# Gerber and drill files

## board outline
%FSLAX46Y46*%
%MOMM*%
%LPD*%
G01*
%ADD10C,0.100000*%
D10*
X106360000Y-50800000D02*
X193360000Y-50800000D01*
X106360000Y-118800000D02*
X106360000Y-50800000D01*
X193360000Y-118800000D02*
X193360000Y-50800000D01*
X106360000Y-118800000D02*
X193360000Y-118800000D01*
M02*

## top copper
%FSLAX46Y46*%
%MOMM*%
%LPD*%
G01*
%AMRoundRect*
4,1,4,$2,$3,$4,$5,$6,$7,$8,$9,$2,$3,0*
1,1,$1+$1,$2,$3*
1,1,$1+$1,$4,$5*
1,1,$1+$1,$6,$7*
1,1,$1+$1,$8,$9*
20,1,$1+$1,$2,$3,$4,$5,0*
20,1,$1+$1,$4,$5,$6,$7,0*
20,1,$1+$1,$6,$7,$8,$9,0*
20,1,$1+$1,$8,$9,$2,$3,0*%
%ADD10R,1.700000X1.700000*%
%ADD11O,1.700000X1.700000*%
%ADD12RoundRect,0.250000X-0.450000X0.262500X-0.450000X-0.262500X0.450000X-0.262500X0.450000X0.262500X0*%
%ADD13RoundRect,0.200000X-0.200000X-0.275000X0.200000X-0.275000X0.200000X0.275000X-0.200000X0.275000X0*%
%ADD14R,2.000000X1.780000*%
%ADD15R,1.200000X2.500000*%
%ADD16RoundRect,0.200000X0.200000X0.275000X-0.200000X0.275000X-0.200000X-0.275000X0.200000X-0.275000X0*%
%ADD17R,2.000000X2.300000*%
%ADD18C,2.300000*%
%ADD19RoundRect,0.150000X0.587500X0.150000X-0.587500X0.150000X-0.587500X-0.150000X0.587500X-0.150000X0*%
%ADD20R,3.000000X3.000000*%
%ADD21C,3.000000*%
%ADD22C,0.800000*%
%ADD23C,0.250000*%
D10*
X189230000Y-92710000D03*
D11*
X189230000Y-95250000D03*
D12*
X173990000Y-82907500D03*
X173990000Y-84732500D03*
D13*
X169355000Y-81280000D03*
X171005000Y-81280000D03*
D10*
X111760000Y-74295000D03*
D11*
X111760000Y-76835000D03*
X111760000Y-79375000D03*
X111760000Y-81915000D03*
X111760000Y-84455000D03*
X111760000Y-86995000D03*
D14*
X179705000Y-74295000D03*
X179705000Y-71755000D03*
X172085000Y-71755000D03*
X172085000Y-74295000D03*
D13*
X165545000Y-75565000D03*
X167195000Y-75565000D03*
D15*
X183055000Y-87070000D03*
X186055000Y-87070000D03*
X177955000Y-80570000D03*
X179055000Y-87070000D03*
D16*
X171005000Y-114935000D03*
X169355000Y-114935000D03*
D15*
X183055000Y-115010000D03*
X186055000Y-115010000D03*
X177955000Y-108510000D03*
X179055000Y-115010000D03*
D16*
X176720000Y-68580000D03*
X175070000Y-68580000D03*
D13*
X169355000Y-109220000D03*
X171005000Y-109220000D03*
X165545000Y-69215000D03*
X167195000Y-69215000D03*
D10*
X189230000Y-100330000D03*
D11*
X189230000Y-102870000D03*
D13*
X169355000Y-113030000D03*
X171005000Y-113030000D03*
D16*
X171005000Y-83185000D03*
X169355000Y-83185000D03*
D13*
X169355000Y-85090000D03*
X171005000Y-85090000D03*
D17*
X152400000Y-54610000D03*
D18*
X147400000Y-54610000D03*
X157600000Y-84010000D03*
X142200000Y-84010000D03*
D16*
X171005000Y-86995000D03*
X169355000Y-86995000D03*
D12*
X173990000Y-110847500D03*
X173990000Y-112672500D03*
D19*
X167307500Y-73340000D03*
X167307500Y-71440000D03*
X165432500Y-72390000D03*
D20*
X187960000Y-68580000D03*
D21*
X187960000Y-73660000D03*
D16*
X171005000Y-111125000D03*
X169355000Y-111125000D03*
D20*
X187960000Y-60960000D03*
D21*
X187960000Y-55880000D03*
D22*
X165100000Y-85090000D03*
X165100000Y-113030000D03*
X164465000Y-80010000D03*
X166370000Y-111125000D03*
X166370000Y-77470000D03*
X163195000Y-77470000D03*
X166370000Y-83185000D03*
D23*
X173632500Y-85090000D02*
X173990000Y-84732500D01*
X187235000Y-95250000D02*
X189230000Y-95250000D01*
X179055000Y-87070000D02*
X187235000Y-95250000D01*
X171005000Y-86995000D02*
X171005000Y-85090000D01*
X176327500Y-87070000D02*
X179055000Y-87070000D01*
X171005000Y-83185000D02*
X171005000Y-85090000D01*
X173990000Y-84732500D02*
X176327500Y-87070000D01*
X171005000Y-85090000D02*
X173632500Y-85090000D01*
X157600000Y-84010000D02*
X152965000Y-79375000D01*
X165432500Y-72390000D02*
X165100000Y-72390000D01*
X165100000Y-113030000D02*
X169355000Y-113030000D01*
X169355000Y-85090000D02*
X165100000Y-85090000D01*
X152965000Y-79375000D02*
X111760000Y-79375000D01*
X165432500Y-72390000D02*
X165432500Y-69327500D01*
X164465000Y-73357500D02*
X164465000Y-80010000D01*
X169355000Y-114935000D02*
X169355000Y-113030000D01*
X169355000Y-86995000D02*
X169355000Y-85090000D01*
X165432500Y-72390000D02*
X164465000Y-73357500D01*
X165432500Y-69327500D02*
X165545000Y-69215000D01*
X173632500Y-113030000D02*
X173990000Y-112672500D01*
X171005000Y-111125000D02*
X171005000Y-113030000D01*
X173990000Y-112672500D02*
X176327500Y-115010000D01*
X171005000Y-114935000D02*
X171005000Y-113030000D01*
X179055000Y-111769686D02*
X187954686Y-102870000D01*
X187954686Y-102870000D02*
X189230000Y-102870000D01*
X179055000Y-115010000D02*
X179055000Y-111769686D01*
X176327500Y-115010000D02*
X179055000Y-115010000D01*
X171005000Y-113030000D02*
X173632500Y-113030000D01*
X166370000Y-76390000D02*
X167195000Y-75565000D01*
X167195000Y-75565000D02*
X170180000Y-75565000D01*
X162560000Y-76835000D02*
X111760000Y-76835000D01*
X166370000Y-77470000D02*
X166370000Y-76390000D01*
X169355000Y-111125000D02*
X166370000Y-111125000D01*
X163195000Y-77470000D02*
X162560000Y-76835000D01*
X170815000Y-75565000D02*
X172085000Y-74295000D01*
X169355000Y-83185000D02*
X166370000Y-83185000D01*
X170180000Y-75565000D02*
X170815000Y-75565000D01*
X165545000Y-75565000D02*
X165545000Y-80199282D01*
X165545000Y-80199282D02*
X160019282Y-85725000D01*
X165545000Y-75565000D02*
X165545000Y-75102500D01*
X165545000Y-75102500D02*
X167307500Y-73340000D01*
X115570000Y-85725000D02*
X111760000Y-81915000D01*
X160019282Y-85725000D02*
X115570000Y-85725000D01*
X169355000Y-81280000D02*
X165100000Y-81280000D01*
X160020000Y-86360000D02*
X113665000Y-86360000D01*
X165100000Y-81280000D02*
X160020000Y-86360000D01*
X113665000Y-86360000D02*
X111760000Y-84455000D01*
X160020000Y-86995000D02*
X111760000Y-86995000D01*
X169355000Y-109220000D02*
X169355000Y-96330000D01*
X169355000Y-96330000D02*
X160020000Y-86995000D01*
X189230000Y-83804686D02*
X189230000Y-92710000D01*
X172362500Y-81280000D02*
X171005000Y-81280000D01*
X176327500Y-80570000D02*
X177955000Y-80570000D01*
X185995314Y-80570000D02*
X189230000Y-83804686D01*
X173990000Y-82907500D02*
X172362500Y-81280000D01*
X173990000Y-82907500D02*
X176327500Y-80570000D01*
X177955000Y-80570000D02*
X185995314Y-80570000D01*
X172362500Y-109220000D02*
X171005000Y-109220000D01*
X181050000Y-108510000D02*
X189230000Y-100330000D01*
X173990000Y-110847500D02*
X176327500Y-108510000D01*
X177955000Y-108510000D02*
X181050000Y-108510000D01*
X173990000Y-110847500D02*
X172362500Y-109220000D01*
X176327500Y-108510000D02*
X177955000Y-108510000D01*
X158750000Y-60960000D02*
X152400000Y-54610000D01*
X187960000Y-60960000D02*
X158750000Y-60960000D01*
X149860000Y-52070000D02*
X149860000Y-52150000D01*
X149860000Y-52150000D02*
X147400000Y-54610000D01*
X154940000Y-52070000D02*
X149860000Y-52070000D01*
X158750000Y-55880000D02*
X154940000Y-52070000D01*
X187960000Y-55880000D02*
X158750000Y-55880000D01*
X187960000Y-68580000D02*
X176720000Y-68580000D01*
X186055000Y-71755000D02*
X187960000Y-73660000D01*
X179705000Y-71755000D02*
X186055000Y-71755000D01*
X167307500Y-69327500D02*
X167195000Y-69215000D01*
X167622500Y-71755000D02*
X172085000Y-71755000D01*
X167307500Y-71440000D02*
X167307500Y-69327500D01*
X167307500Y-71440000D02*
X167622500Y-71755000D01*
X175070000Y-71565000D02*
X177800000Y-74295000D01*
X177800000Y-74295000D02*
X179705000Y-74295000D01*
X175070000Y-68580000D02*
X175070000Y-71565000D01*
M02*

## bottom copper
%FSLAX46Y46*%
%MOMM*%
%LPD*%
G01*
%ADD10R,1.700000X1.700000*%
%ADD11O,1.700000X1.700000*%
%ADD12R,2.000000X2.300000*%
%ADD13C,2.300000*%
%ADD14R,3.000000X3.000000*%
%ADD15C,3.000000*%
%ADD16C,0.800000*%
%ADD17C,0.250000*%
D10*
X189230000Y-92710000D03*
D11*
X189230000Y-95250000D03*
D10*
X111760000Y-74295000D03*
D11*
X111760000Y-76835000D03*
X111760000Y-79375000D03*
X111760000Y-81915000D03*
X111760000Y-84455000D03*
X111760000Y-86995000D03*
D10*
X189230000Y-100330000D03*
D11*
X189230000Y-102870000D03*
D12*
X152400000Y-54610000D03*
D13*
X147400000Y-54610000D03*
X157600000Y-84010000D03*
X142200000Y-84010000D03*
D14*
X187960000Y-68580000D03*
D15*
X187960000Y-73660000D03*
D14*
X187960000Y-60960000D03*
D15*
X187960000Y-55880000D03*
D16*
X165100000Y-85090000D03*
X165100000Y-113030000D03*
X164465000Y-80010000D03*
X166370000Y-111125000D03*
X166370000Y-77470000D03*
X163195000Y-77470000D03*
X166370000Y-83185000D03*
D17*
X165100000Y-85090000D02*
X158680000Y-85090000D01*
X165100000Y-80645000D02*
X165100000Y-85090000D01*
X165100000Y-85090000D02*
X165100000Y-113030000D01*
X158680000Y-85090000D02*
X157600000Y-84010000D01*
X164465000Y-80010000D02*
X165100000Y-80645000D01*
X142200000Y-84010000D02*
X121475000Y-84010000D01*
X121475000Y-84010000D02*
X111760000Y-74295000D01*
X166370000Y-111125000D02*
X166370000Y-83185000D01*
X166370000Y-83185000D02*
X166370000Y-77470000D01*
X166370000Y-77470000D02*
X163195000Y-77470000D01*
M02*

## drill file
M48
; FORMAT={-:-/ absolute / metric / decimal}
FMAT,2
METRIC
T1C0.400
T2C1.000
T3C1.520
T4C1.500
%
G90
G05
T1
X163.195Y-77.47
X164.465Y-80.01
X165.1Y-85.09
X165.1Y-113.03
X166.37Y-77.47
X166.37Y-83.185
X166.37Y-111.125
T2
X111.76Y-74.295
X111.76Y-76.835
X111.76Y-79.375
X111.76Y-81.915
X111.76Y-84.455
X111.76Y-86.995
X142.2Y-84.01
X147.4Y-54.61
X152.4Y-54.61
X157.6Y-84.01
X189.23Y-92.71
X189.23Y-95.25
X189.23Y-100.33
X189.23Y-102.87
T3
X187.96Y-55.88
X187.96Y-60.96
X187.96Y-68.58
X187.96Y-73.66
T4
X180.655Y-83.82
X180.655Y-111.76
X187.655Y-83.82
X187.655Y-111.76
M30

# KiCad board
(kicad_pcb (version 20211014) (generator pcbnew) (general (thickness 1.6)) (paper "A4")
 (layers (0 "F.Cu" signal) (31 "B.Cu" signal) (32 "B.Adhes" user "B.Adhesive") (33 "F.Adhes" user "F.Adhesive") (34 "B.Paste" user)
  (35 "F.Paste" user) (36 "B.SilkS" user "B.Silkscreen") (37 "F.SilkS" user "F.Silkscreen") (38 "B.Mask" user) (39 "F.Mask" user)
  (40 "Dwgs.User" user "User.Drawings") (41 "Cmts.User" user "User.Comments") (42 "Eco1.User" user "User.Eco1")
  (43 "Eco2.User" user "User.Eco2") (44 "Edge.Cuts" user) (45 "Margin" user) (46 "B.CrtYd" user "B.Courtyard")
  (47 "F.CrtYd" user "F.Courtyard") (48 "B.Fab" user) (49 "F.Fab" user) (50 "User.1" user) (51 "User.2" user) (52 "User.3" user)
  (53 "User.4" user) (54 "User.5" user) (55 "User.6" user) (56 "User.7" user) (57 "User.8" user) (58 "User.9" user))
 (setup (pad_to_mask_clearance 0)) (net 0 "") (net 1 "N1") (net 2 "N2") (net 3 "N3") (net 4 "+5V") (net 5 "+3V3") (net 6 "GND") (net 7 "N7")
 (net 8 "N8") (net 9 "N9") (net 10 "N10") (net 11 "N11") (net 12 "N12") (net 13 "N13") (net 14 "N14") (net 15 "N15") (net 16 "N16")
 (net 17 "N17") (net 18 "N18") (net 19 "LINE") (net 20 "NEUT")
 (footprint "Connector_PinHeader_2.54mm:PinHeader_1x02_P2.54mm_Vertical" (layer "F.Cu") (at 189.23 92.71)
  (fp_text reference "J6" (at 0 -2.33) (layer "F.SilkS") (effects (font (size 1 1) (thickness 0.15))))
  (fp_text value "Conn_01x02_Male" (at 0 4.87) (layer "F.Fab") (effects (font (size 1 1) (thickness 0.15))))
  (pad "1" thru_hole rect locked (at 0 0) (size 1.7 1.7) (drill 1) (layers *.Cu *.Mask) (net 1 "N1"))
  (pad "2" thru_hole oval locked (at 0 2.54) (size 1.7 1.7) (drill 1) (layers *.Cu *.Mask) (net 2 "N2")))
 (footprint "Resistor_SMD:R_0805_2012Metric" (layer "F.Cu") (at 173.99 83.82 -90)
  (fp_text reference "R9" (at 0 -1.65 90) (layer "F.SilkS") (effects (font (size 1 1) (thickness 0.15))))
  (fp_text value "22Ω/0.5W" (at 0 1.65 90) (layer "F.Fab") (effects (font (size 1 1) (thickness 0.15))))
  (pad "1" smd roundrect locked (at -0.9125 0 270) (size 1.025 1.4) (layers "F.Cu" "F.Paste" "F.Mask") (roundrect_rratio 0.243902)
   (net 1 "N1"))
  (pad "2" smd roundrect locked (at 0.9125 0 270) (size 1.025 1.4) (layers "F.Cu" "F.Paste" "F.Mask") (roundrect_rratio 0.243902)
   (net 2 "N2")))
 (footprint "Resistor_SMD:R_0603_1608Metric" (layer "F.Cu") (at 170.18 81.28)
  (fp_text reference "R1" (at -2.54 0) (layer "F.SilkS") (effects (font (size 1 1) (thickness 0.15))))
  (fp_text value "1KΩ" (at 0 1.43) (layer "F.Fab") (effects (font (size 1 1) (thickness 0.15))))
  (pad "1" smd roundrect locked (at -0.825 0) (size 0.8 0.95) (layers "F.Cu" "F.Paste" "F.Mask") (roundrect_rratio 0.25) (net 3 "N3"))
  (pad "2" smd roundrect locked (at 0.825 0) (size 0.8 0.95) (layers "F.Cu" "F.Paste" "F.Mask") (roundrect_rratio 0.25) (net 1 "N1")))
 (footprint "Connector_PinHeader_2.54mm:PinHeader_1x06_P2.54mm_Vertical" (layer "F.Cu") (at 111.76 74.295)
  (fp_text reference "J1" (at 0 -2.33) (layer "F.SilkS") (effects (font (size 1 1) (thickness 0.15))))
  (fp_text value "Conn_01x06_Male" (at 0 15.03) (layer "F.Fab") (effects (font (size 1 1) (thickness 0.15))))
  (pad "1" thru_hole rect locked (at 0 0) (size 1.7 1.7) (drill 1) (layers *.Cu *.Mask) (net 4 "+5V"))
  (pad "2" thru_hole oval locked (at 0 2.54) (size 1.7 1.7) (drill 1) (layers *.Cu *.Mask) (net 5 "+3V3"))
  (pad "3" thru_hole oval locked (at 0 5.08) (size 1.7 1.7) (drill 1) (layers *.Cu *.Mask) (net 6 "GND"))
  (pad "4" thru_hole oval locked (at 0 7.62) (size 1.7 1.7) (drill 1) (layers *.Cu *.Mask) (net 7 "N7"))
  (pad "5" thru_hole oval locked (at 0 10.16) (size 1.7 1.7) (drill 1) (layers *.Cu *.Mask) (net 3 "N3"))
  (pad "6" thru_hole oval locked (at 0 12.7) (size 1.7 1.7) (drill 1) (layers *.Cu *.Mask) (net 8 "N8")))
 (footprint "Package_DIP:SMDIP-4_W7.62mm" (layer "F.Cu") (at 175.895 73.025 180)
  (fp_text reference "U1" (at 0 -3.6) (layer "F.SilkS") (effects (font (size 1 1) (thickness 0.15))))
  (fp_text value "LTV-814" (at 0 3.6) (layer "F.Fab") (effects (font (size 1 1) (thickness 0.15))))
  (pad "1" smd rect locked (at -3.81 -1.27 180) (size 2 1.78) (layers "F.Cu" "F.Paste" "F.Mask") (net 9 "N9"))
  (pad "2" smd rect locked (at -3.81 1.27 180) (size 2 1.78) (layers "F.Cu" "F.Paste" "F.Mask") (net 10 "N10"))
  (pad "3" smd rect locked (at 3.81 1.27 180) (size 2 1.78) (layers "F.Cu" "F.Paste" "F.Mask") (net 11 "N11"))
  (pad "4" smd rect locked (at 3.81 -1.27 180) (size 2 1.78) (layers "F.Cu" "F.Paste" "F.Mask") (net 5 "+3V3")))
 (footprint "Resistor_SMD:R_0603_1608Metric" (layer "F.Cu") (at 166.37 75.565)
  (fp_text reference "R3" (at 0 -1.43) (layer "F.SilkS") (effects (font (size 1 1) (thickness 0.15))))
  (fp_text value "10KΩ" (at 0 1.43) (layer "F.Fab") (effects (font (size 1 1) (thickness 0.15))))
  (pad "1" smd roundrect locked (at -0.825 0) (size 0.8 0.95) (layers "F.Cu" "F.Paste" "F.Mask") (roundrect_rratio 0.25) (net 7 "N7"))
  (pad "2" smd roundrect locked (at 0.825 0) (size 0.8 0.95) (layers "F.Cu" "F.Paste" "F.Mask") (roundrect_rratio 0.25) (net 5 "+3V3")))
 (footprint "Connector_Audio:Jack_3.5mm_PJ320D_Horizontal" (layer "F.Cu") (at 182.88 83.82 180)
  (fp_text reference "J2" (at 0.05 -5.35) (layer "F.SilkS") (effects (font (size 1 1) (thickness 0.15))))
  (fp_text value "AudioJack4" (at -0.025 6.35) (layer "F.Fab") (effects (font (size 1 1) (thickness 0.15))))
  (pad "" np_thru_hole circle locked (at 2.225 0 180) (size 1.5 1.5) (drill 1.5) (layers *.Cu *.Mask))
  (pad "" np_thru_hole circle locked (at -4.775 0 180) (size 1.5 1.5) (drill 1.5) (layers *.Cu *.Mask))
  (pad "R1" smd rect locked (at -0.175 -3.25 180) (size 1.2 2.5) (layers "F.Cu" "F.Paste" "F.Mask") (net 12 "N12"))
  (pad "R2" smd rect locked (at -3.175 -3.25 180) (size 1.2 2.5) (layers "F.Cu" "F.Paste" "F.Mask") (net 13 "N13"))
  (pad "S" smd rect locked (at 4.925 3.25 180) (size 1.2 2.5) (layers "F.Cu" "F.Paste" "F.Mask") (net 1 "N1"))
  (pad "T" smd rect locked (at 3.825 -3.25 180) (size 1.2 2.5) (layers "F.Cu" "F.Paste" "F.Mask") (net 2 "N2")))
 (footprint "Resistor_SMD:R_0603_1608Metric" (layer "F.Cu") (at 170.18 114.935 180)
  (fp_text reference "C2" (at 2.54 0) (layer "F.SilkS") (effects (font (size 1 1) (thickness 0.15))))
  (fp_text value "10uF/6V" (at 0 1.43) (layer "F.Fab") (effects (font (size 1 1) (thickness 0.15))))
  (pad "1" smd roundrect locked (at -0.825 0 180) (size 0.8 0.95) (layers "F.Cu" "F.Paste" "F.Mask") (roundrect_rratio 0.25) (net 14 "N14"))
  (pad "2" smd roundrect locked (at 0.825 0 180) (size 0.8 0.95) (layers "F.Cu" "F.Paste" "F.Mask") (roundrect_rratio 0.25) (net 6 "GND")))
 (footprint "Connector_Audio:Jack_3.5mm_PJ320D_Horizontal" (layer "F.Cu") (at 182.88 111.76 180)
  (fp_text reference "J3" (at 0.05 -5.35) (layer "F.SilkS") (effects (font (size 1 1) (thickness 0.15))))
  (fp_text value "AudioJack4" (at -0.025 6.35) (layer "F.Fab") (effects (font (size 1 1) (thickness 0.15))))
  (pad "" np_thru_hole circle locked (at 2.225 0 180) (size 1.5 1.5) (drill 1.5) (layers *.Cu *.Mask))
  (pad "" np_thru_hole circle locked (at -4.775 0 180) (size 1.5 1.5) (drill 1.5) (layers *.Cu *.Mask))
  (pad "R1" smd rect locked (at -0.175 -3.25 180) (size 1.2 2.5) (layers "F.Cu" "F.Paste" "F.Mask") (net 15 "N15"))
  (pad "R2" smd rect locked (at -3.175 -3.25 180) (size 1.2 2.5) (layers "F.Cu" "F.Paste" "F.Mask") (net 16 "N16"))
  (pad "S" smd rect locked (at 4.925 3.25 180) (size 1.2 2.5) (layers "F.Cu" "F.Paste" "F.Mask") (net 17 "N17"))
  (pad "T" smd rect locked (at 3.825 -3.25 180) (size 1.2 2.5) (layers "F.Cu" "F.Paste" "F.Mask") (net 14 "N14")))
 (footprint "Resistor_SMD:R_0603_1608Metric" (layer "F.Cu") (at 175.895 68.58 180)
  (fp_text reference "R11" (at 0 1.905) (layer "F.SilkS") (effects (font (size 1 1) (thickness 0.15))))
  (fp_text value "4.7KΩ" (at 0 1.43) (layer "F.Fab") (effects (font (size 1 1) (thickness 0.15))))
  (pad "1" smd roundrect locked (at -0.825 0 180) (size 0.8 0.95) (layers "F.Cu" "F.Paste" "F.Mask") (roundrect_rratio 0.25) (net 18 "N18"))
  (pad "2" smd roundrect locked (at 0.825 0 180) (size 0.8 0.95) (layers "F.Cu" "F.Paste" "F.Mask") (roundrect_rratio 0.25) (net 9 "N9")))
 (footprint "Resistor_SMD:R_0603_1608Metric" (layer "F.Cu") (at 170.18 109.22)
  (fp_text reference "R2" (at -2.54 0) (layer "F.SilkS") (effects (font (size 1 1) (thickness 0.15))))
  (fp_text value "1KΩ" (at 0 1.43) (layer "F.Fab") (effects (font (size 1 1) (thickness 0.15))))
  (pad "1" smd roundrect locked (at -0.825 0) (size 0.8 0.95) (layers "F.Cu" "F.Paste" "F.Mask") (roundrect_rratio 0.25) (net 8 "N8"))
  (pad "2" smd roundrect locked (at 0.825 0) (size 0.8 0.95) (layers "F.Cu" "F.Paste" "F.Mask") (roundrect_rratio 0.25) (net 17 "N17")))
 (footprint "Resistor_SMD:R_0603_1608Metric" (layer "F.Cu") (at 166.37 69.215)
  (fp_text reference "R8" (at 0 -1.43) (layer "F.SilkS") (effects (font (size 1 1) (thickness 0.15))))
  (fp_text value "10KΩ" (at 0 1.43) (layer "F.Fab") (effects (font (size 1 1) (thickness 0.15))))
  (pad "1" smd roundrect locked (at -0.825 0) (size 0.8 0.95) (layers "F.Cu" "F.Paste" "F.Mask") (roundrect_rratio 0.25) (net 6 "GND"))
  (pad "2" smd roundrect locked (at 0.825 0) (size 0.8 0.95) (layers "F.Cu" "F.Paste" "F.Mask") (roundrect_rratio 0.25) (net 11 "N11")))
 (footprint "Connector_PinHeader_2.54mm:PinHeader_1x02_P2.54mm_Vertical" (layer "F.Cu") (at 189.23 100.33)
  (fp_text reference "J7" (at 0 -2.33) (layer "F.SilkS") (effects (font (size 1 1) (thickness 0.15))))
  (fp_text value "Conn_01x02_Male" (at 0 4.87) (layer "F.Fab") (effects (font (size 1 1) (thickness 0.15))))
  (pad "1" thru_hole rect locked (at 0 0) (size 1.7 1.7) (drill 1) (layers *.Cu *.Mask) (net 17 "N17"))
  (pad "2" thru_hole oval locked (at 0 2.54) (size 1.7 1.7) (drill 1) (layers *.Cu *.Mask) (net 14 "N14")))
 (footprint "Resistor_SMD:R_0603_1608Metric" (layer "F.Cu") (at 170.18 113.03)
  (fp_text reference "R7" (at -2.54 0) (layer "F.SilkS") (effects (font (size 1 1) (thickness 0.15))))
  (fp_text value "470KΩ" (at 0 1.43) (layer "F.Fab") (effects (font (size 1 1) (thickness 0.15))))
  (pad "1" smd roundrect locked (at -0.825 0) (size 0.8 0.95) (layers "F.Cu" "F.Paste" "F.Mask") (roundrect_rratio 0.25) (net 6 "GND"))
  (pad "2" smd roundrect locked (at 0.825 0) (size 0.8 0.95) (layers "F.Cu" "F.Paste" "F.Mask") (roundrect_rratio 0.25) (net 14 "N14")))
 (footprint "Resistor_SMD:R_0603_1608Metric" (layer "F.Cu") (at 170.18 83.185 180)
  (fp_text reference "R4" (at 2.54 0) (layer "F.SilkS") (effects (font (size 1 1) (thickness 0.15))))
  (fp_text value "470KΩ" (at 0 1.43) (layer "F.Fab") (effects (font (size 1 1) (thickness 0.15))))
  (pad "1" smd roundrect locked (at -0.825 0 180) (size 0.8 0.95) (layers "F.Cu" "F.Paste" "F.Mask") (roundrect_rratio 0.25) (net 2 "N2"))
  (pad "2" smd roundrect locked (at 0.825 0 180) (size 0.8 0.95) (layers "F.Cu" "F.Paste" "F.Mask") (roundrect_rratio 0.25) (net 5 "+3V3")))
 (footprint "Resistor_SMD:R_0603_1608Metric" (layer "F.Cu") (at 170.18 85.09)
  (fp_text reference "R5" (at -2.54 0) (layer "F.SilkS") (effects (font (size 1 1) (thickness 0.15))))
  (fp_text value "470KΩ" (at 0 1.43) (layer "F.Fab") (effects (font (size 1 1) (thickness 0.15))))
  (pad "1" smd roundrect locked (at -0.825 0) (size 0.8 0.95) (layers "F.Cu" "F.Paste" "F.Mask") (roundrect_rratio 0.25) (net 6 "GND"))
  (pad "2" smd roundrect locked (at 0.825 0) (size 0.8 0.95) (layers "F.Cu" "F.Paste" "F.Mask") (roundrect_rratio 0.25) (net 2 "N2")))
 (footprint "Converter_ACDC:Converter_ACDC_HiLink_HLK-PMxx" (layer "F.Cu") (at 152.4 54.61 -90)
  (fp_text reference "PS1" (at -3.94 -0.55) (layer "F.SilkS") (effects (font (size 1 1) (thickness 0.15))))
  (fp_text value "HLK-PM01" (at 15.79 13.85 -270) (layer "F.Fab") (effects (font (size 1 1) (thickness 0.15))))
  (pad "1" thru_hole rect locked (at 0 0 270) (size 2.3 2) (drill 1) (layers *.Cu *.Mask) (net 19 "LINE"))
  (pad "2" thru_hole circle locked (at 0 5 270) (size 2.3 2.3) (drill 1) (layers *.Cu *.Mask) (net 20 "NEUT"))
  (pad "3" thru_hole circle locked (at 29.4 -5.2 270) (size 2.3 2.3) (drill 1) (layers *.Cu *.Mask) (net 6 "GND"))
  (pad "4" thru_hole circle locked (at 29.4 10.2 270) (size 2.3 2.3) (drill 1) (layers *.Cu *.Mask) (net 4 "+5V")))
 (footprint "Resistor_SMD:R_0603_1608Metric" (layer "F.Cu") (at 170.18 86.995 180)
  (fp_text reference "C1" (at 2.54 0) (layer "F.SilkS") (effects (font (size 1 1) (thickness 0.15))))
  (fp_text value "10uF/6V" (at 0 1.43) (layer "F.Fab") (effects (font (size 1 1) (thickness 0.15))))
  (pad "1" smd roundrect locked (at -0.825 0 180) (size 0.8 0.95) (layers "F.Cu" "F.Paste" "F.Mask") (roundrect_rratio 0.25) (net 2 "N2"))
  (pad "2" smd roundrect locked (at 0.825 0 180) (size 0.8 0.95) (layers "F.Cu" "F.Paste" "F.Mask") (roundrect_rratio 0.25) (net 6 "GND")))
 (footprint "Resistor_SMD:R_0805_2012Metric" (layer "F.Cu") (at 173.99 111.76 -90)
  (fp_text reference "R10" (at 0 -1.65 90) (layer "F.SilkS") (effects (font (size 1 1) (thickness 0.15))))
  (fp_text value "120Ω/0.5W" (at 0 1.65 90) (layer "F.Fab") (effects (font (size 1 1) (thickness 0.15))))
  (pad "1" smd roundrect locked (at -0.9125 0 270) (size 1.025 1.4) (layers "F.Cu" "F.Paste" "F.Mask") (roundrect_rratio 0.243902)
   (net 17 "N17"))
  (pad "2" smd roundrect locked (at 0.9125 0 270) (size 1.025 1.4) (layers "F.Cu" "F.Paste" "F.Mask") (roundrect_rratio 0.243902)
   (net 14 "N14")))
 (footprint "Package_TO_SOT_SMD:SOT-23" (layer "F.Cu") (at 166.37 72.39 180)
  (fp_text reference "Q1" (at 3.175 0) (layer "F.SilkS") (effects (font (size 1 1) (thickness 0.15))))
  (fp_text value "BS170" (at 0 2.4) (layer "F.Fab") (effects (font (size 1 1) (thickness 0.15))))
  (pad "1" smd roundrect locked (at -0.9375 -0.95 180) (size 1.475 0.6) (layers "F.Cu" "F.Paste" "F.Mask") (roundrect_rratio 0.25)
   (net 7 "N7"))
  (pad "2" smd roundrect locked (at -0.9375 0.95 180) (size 1.475 0.6) (layers "F.Cu" "F.Paste" "F.Mask") (roundrect_rratio 0.25)
   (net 11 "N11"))
  (pad "3" smd roundrect locked (at 0.9375 0 180) (size 1.475 0.6) (layers "F.Cu" "F.Paste" "F.Mask") (roundrect_rratio 0.25) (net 6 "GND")))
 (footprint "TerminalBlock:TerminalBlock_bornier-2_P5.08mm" (layer "F.Cu") (at 187.96 68.58 -90)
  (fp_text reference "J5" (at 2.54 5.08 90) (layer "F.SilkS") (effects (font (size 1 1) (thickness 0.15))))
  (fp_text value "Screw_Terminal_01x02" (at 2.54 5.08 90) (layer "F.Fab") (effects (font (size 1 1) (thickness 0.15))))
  (pad "1" thru_hole rect locked (at 0 0 270) (size 3 3) (drill 1.52) (layers *.Cu *.Mask) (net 18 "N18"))
  (pad "2" thru_hole circle locked (at 5.08 0 270) (size 3 3) (drill 1.52) (layers *.Cu *.Mask) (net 10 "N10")))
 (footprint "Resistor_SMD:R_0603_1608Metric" (layer "F.Cu") (at 170.18 111.125 180)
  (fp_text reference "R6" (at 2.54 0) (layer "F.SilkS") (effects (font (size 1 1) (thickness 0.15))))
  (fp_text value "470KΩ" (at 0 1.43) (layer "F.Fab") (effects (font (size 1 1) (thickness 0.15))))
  (pad "1" smd roundrect locked (at -0.825 0 180) (size 0.8 0.95) (layers "F.Cu" "F.Paste" "F.Mask") (roundrect_rratio 0.25) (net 14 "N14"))
  (pad "2" smd roundrect locked (at 0.825 0 180) (size 0.8 0.95) (layers "F.Cu" "F.Paste" "F.Mask") (roundrect_rratio 0.25) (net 5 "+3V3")))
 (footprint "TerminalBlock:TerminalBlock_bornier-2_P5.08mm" (layer "F.Cu") (at 187.96 60.96 90)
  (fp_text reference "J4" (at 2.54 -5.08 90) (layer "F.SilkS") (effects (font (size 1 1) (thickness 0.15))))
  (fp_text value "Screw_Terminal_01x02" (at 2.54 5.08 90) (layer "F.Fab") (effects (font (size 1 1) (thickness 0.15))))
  (pad "1" thru_hole rect locked (at 0 0 90) (size 3 3) (drill 1.52) (layers *.Cu *.Mask) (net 19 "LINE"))
  (pad "2" thru_hole circle locked (at 5.08 0 90) (size 3 3) (drill 1.52) (layers *.Cu *.Mask) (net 20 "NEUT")))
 (gr_line locked (start 106.36 50.8) (end 193.36 50.8) (layer "Edge.Cuts") (width 0.1))
 (gr_line locked (start 106.36 118.8) (end 106.36 50.8) (layer "Edge.Cuts") (width 0.1))
 (gr_line locked (start 193.36 118.8) (end 193.36 50.8) (layer "Edge.Cuts") (width 0.1))
 (gr_line locked (start 106.36 118.8) (end 193.36 118.8) (layer "Edge.Cuts") (width 0.1))
 (segment (start 173.6325 85.09) (end 173.99 84.7325) (width 0.25) (layer "F.Cu") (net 2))
 (segment (start 187.235 95.25) (end 189.23 95.25) (width 0.25) (layer "F.Cu") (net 2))
 (segment (start 179.055 87.07) (end 187.235 95.25) (width 0.25) (layer "F.Cu") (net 2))
 (segment (start 171.005 86.995) (end 171.005 85.09) (width 0.25) (layer "F.Cu") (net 2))
 (segment (start 176.3275 87.07) (end 179.055 87.07) (width 0.25) (layer "F.Cu") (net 2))
 (segment (start 171.005 83.185) (end 171.005 85.09) (width 0.25) (layer "F.Cu") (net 2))
 (segment (start 173.99 84.7325) (end 176.3275 87.07) (width 0.25) (layer "F.Cu") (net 2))
 (segment (start 171.005 85.09) (end 173.6325 85.09) (width 0.25) (layer "F.Cu") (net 2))
 (segment (start 157.6 84.01) (end 152.965 79.375) (width 0.25) (layer "F.Cu") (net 6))
 (segment (start 165.4325 72.39) (end 165.1 72.39) (width 0.25) (layer "F.Cu") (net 6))
 (segment (start 165.1 113.03) (end 169.355 113.03) (width 0.25) (layer "F.Cu") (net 6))
 (segment (start 169.355 85.09) (end 165.1 85.09) (width 0.25) (layer "F.Cu") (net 6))
 (segment (start 152.965 79.375) (end 111.76 79.375) (width 0.25) (layer "F.Cu") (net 6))
 (segment (start 165.4325 72.39) (end 165.4325 69.3275) (width 0.25) (layer "F.Cu") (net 6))
 (segment (start 164.465 73.3575) (end 164.465 80.01) (width 0.25) (layer "F.Cu") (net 6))
 (segment (start 169.355 114.935) (end 169.355 113.03) (width 0.25) (layer "F.Cu") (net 6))
 (segment (start 169.355 86.995) (end 169.355 85.09) (width 0.25) (layer "F.Cu") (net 6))
 (segment (start 165.4325 72.39) (end 164.465 73.3575) (width 0.25) (layer "F.Cu") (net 6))
 (segment (start 165.4325 69.3275) (end 165.545 69.215) (width 0.25) (layer "F.Cu") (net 6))
 (via (at 165.1 85.09) (size 0.8) (drill 0.4) (layers "F.Cu" "B.Cu") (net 6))
 (via (at 165.1 113.03) (size 0.8) (drill 0.4) (layers "F.Cu" "B.Cu") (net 6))
 (via (at 164.465 80.01) (size 0.8) (drill 0.4) (layers "F.Cu" "B.Cu") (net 6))
 (segment (start 165.1 85.09) (end 158.68 85.09) (width 0.25) (layer "B.Cu") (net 6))
 (segment (start 165.1 80.645) (end 165.1 85.09) (width 0.25) (layer "B.Cu") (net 6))
 (segment (start 165.1 85.09) (end 165.1 113.03) (width 0.25) (layer "B.Cu") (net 6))
 (segment (start 158.68 85.09) (end 157.6 84.01) (width 0.25) (layer "B.Cu") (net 6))
 (segment (start 164.465 80.01) (end 165.1 80.645) (width 0.25) (layer "B.Cu") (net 6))
 (segment (start 173.6325 113.03) (end 173.99 112.6725) (width 0.25) (layer "F.Cu") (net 14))
 (segment (start 171.005 111.125) (end 171.005 113.03) (width 0.25) (layer "F.Cu") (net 14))
 (segment (start 173.99 112.6725) (end 176.3275 115.01) (width 0.25) (layer "F.Cu") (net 14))
 (segment (start 171.005 114.935) (end 171.005 113.03) (width 0.25) (layer "F.Cu") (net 14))
 (segment (start 179.055 111.769686) (end 187.954686 102.87) (width 0.25) (layer "F.Cu") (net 14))
 (segment (start 187.954686 102.87) (end 189.23 102.87) (width 0.25) (layer "F.Cu") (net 14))
 (segment (start 179.055 115.01) (end 179.055 111.769686) (width 0.25) (layer "F.Cu") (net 14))
 (segment (start 176.3275 115.01) (end 179.055 115.01) (width 0.25) (layer "F.Cu") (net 14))
 (segment (start 171.005 113.03) (end 173.6325 113.03) (width 0.25) (layer "F.Cu") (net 14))
 (segment (start 142.2 84.01) (end 121.475 84.01) (width 0.25) (layer "B.Cu") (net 4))
 (segment (start 121.475 84.01) (end 111.76 74.295) (width 0.25) (layer "B.Cu") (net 4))
 (segment (start 166.37 76.39) (end 167.195 75.565) (width 0.25) (layer "F.Cu") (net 5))
 (segment (start 167.195 75.565) (end 170.18 75.565) (width 0.25) (layer "F.Cu") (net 5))
 (segment (start 162.56 76.835) (end 111.76 76.835) (width 0.25) (layer "F.Cu") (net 5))
 (segment (start 166.37 77.47) (end 166.37 76.39) (width 0.25) (layer "F.Cu") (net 5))
 (segment (start 169.355 111.125) (end 166.37 111.125) (width 0.25) (layer "F.Cu") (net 5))
 (segment (start 163.195 77.47) (end 162.56 76.835) (width 0.25) (layer "F.Cu") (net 5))
 (segment (start 170.815 75.565) (end 172.085 74.295) (width 0.25) (layer "F.Cu") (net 5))
 (segment (start 169.355 83.185) (end 166.37 83.185) (width 0.25) (layer "F.Cu") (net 5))
 (segment (start 170.18 75.565) (end 170.815 75.565) (width 0.25) (layer "F.Cu") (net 5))
 (via (at 166.37 111.125) (size 0.8) (drill 0.4) (layers "F.Cu" "B.Cu") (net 5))
 (via (at 166.37 77.47) (size 0.8) (drill 0.4) (layers "F.Cu" "B.Cu") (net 5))
 (via (at 163.195 77.47) (size 0.8) (drill 0.4) (layers "F.Cu" "B.Cu") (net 5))
 (via (at 166.37 83.185) (size 0.8) (drill 0.4) (layers "F.Cu" "B.Cu") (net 5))
 (segment (start 166.37 111.125) (end 166.37 83.185) (width 0.25) (layer "B.Cu") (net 5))
 (segment (start 166.37 83.185) (end 166.37 77.47) (width 0.25) (layer "B.Cu") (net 5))
 (segment (start 166.37 77.47) (end 163.195 77.47) (width 0.25) (layer "B.Cu") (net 5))
 (segment (start 165.545 75.565) (end 165.545 80.199282) (width 0.25) (layer "F.Cu") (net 7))
 (segment (start 165.545 80.199282) (end 160.019282 85.725) (width 0.25) (layer "F.Cu") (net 7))
 (segment (start 165.545 75.565) (end 165.545 75.1025) (width 0.25) (layer "F.Cu") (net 7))
 (segment (start 165.545 75.1025) (end 167.3075 73.34) (width 0.25) (layer "F.Cu") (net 7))
 (segment (start 115.57 85.725) (end 111.76 81.915) (width 0.25) (layer "F.Cu") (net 7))
 (segment (start 160.019282 85.725) (end 115.57 85.725) (width 0.25) (layer "F.Cu") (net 7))
 (segment (start 169.355 81.28) (end 165.1 81.28) (width 0.25) (layer "F.Cu") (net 3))
 (segment (start 160.02 86.36) (end 113.665 86.36) (width 0.25) (layer "F.Cu") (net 3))
 (segment (start 165.1 81.28) (end 160.02 86.36) (width 0.25) (layer "F.Cu") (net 3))
 (segment (start 113.665 86.36) (end 111.76 84.455) (width 0.25) (layer "F.Cu") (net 3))
 (segment (start 160.02 86.995) (end 111.76 86.995) (width 0.25) (layer "F.Cu") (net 8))
 (segment (start 169.355 109.22) (end 169.355 96.33) (width 0.25) (layer "F.Cu") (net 8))
 (segment (start 169.355 96.33) (end 160.02 86.995) (width 0.25) (layer "F.Cu") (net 8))
 (segment (start 189.23 83.804686) (end 189.23 92.71) (width 0.25) (layer "F.Cu") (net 1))
 (segment (start 172.3625 81.28) (end 171.005 81.28) (width 0.25) (layer "F.Cu") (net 1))
 (segment (start 176.3275 80.57) (end 177.955 80.57) (width 0.25) (layer "F.Cu") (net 1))
 (segment (start 185.995314 80.57) (end 189.23 83.804686) (width 0.25) (layer "F.Cu") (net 1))
 (segment (start 173.99 82.9075) (end 172.3625 81.28) (width 0.25) (layer "F.Cu") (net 1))
 (segment (start 173.99 82.9075) (end 176.3275 80.57) (width 0.25) (layer "F.Cu") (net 1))
 (segment (start 177.955 80.57) (end 185.995314 80.57) (width 0.25) (layer "F.Cu") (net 1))
 (segment (start 172.3625 109.22) (end 171.005 109.22) (width 0.25) (layer "F.Cu") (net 17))
 (segment (start 181.05 108.51) (end 189.23 100.33) (width 0.25) (layer "F.Cu") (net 17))
 (segment (start 173.99 110.8475) (end 176.3275 108.51) (width 0.25) (layer "F.Cu") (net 17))
 (segment (start 177.955 108.51) (end 181.05 108.51) (width 0.25) (layer "F.Cu") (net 17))
 (segment (start 173.99 110.8475) (end 172.3625 109.22) (width 0.25) (layer "F.Cu") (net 17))
 (segment (start 176.3275 108.51) (end 177.955 108.51) (width 0.25) (layer "F.Cu") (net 17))
 (segment (start 158.75 60.96) (end 152.4 54.61) (width 0.25) (layer "F.Cu") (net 19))
 (segment (start 187.96 60.96) (end 158.75 60.96) (width 0.25) (layer "F.Cu") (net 19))
 (segment (start 149.86 52.07) (end 149.86 52.15) (width 0.25) (layer "F.Cu") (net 20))
 (segment (start 149.86 52.15) (end 147.4 54.61) (width 0.25) (layer "F.Cu") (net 20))
 (segment (start 154.94 52.07) (end 149.86 52.07) (width 0.25) (layer "F.Cu") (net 20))
 (segment (start 158.75 55.88) (end 154.94 52.07) (width 0.25) (layer "F.Cu") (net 20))
 (segment (start 187.96 55.88) (end 158.75 55.88) (width 0.25) (layer "F.Cu") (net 20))
 (segment (start 187.96 68.58) (end 176.72 68.58) (width 0.25) (layer "F.Cu") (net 18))
 (segment (start 186.055 71.755) (end 187.96 73.66) (width 0.25) (layer "F.Cu") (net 10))
 (segment (start 179.705 71.755) (end 186.055 71.755) (width 0.25) (layer "F.Cu") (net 10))
 (segment (start 167.3075 69.3275) (end 167.195 69.215) (width 0.25) (layer "F.Cu") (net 11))
 (segment (start 167.6225 71.755) (end 172.085 71.755) (width 0.25) (layer "F.Cu") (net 11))
 (segment (start 167.3075 71.44) (end 167.3075 69.3275) (width 0.25) (layer "F.Cu") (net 11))
 (segment (start 167.3075 71.44) (end 167.6225 71.755) (width 0.25) (layer "F.Cu") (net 11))
 (segment (start 175.07 71.565) (end 177.8 74.295) (width 0.25) (layer "F.Cu") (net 9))
 (segment (start 177.8 74.295) (end 179.705 74.295) (width 0.25) (layer "F.Cu") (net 9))
 (segment (start 175.07 68.58) (end 175.07 71.565) (width 0.25) (layer "F.Cu") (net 9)))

